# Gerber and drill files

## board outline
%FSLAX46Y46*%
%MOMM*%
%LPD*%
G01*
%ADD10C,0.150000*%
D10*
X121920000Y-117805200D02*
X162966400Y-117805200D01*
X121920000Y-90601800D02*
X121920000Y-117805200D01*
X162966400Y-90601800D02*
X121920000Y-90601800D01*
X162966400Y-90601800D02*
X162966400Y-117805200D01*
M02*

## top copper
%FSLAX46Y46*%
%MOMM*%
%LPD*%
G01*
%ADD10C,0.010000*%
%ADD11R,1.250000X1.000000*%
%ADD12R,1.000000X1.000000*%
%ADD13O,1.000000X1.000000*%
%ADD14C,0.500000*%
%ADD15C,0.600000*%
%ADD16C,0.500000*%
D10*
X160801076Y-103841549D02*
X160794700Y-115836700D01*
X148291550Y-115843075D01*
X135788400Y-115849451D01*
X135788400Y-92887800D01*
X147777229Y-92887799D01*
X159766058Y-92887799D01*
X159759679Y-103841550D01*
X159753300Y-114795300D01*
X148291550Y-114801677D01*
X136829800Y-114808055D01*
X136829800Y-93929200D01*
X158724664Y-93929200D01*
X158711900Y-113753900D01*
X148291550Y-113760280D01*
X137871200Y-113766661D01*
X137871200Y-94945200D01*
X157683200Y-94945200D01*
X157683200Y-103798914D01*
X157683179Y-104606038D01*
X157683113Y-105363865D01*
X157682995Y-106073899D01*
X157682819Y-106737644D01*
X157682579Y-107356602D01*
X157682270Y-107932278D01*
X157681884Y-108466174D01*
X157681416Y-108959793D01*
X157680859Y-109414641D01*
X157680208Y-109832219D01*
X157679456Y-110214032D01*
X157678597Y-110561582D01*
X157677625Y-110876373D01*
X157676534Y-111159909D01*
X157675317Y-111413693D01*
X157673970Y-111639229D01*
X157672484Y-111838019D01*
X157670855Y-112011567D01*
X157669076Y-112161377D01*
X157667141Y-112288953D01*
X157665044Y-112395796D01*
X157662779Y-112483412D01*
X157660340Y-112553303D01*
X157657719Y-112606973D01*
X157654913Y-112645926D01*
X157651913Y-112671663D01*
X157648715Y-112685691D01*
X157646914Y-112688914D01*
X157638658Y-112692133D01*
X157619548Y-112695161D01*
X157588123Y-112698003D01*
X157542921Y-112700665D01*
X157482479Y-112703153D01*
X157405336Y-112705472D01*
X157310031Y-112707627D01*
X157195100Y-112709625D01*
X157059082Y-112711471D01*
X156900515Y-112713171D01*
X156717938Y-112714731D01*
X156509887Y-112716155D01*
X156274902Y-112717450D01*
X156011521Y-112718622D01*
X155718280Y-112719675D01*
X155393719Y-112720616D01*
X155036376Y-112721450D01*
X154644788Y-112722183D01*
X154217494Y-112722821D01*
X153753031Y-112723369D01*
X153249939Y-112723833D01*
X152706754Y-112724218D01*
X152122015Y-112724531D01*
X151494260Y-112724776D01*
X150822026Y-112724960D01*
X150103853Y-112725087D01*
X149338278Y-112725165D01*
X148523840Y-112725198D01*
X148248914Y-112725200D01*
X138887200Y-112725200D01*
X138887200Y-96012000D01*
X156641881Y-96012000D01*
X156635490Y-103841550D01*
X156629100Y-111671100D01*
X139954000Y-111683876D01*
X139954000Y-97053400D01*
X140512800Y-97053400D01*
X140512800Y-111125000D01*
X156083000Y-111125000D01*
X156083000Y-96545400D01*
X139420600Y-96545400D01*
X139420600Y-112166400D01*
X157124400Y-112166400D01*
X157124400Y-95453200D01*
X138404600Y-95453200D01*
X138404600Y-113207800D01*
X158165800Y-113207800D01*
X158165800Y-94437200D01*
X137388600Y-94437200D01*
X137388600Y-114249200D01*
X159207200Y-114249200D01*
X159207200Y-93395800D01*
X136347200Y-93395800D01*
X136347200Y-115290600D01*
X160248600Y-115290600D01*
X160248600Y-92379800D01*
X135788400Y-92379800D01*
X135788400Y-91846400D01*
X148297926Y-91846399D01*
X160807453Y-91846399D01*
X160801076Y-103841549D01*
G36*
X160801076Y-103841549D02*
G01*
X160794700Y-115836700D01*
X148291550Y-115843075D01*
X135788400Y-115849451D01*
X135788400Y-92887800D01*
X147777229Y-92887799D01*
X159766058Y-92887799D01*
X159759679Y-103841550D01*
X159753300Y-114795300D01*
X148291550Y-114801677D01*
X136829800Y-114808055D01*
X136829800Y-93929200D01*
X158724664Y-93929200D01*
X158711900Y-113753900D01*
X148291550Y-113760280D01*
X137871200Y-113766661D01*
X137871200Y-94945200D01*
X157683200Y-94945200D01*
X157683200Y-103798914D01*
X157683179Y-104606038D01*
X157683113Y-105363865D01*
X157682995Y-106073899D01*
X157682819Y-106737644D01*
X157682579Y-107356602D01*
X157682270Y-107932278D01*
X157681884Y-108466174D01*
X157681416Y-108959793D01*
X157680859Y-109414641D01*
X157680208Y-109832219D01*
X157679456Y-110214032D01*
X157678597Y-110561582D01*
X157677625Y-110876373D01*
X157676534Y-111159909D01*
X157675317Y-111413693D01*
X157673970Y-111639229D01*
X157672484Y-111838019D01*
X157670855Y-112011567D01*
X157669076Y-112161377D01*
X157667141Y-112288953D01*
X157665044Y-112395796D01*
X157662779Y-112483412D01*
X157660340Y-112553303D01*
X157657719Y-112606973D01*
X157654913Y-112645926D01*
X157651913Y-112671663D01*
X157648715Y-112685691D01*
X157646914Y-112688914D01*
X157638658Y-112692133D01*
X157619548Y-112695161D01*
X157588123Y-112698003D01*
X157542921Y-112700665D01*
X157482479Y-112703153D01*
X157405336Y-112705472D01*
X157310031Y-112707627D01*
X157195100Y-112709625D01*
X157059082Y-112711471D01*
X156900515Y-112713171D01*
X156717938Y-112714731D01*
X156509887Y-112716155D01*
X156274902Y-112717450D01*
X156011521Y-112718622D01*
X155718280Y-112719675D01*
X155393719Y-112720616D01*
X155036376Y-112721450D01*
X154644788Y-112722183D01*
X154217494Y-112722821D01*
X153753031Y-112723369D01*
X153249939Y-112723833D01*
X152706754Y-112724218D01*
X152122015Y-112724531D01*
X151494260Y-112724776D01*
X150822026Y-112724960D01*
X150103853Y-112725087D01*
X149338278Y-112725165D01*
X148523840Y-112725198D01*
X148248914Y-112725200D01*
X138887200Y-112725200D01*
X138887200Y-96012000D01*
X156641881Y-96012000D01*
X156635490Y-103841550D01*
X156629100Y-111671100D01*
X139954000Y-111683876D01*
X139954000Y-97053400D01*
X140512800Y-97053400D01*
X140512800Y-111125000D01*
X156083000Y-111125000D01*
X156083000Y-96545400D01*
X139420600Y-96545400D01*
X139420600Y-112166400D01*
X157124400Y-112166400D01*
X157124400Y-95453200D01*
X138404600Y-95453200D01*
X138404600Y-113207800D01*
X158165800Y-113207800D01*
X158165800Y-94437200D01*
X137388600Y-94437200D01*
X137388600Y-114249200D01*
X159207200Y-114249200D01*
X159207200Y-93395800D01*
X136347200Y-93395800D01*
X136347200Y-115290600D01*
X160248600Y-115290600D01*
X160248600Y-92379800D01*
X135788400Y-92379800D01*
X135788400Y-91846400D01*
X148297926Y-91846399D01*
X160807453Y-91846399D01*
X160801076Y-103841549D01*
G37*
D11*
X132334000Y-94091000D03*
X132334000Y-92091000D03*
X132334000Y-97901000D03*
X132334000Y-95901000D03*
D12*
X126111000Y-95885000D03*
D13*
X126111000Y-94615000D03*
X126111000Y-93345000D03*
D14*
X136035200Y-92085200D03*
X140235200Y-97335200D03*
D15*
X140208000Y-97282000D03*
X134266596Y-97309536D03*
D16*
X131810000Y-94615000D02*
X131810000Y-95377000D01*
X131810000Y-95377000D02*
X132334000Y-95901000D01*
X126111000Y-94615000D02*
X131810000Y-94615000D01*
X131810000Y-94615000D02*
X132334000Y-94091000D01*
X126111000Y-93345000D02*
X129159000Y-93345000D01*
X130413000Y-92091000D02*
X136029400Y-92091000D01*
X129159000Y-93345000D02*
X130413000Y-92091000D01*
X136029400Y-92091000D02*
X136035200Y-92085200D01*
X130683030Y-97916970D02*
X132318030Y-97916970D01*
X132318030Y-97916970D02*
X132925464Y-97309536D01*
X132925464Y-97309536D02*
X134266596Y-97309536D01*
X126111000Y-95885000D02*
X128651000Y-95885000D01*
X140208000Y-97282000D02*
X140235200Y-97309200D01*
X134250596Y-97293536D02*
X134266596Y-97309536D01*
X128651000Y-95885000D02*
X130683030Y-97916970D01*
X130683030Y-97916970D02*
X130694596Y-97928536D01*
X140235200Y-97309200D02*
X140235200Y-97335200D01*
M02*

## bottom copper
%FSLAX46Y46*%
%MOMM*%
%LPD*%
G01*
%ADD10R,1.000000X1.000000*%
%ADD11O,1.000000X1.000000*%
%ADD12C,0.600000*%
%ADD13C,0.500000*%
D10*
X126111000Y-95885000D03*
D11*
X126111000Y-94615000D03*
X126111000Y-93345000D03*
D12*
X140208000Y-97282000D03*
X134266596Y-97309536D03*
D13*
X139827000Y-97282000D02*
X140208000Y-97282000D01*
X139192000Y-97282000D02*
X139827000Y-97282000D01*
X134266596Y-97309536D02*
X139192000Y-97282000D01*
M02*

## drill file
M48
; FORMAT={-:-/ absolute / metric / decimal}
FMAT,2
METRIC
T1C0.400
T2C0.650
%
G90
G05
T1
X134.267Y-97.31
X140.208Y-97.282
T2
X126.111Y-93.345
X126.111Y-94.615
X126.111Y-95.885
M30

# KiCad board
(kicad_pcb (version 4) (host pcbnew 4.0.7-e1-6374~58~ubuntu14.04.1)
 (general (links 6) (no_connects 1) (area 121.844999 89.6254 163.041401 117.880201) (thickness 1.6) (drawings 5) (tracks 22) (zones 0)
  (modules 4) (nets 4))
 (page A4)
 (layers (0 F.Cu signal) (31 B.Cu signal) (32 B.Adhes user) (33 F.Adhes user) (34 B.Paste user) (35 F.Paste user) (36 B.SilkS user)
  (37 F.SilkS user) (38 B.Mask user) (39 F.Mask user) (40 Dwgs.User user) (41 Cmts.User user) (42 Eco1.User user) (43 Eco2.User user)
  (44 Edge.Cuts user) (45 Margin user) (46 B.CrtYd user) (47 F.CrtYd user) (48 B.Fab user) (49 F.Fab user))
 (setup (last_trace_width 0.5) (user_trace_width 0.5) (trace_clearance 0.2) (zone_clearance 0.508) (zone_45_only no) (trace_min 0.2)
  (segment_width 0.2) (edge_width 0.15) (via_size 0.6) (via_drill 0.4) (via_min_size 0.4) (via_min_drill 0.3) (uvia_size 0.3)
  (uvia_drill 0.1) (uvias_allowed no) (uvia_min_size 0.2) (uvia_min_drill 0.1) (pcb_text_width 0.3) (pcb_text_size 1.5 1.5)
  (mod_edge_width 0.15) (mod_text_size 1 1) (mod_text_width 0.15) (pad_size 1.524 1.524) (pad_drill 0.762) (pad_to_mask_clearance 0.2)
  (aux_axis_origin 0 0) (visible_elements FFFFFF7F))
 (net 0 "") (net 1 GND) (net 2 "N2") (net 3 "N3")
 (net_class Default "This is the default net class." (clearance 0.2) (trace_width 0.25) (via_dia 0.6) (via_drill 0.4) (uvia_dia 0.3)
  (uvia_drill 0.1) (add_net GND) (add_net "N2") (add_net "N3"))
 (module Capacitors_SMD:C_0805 (layer F.Cu) (at 132.334 93.091 90)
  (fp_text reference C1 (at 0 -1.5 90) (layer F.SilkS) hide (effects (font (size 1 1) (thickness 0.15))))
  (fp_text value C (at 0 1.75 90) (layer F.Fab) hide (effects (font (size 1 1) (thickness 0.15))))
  (pad 1 smd rect (at -1 0 90) (size 1 1.25) (layers F.Cu F.Paste F.Mask) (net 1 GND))
  (pad 2 smd rect (at 1 0 90) (size 1 1.25) (layers F.Cu F.Paste F.Mask) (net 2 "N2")))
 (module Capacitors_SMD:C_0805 (layer F.Cu) (at 132.334 96.901 90)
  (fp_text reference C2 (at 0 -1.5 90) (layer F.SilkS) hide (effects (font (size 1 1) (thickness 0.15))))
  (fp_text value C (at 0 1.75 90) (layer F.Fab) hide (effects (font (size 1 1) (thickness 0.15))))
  (pad 1 smd rect (at -1 0 90) (size 1 1.25) (layers F.Cu F.Paste F.Mask) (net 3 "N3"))
  (pad 2 smd rect (at 1 0 90) (size 1 1.25) (layers F.Cu F.Paste F.Mask) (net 1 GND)))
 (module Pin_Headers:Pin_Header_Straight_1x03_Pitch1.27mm (layer F.Cu) (at 126.111 95.885 180)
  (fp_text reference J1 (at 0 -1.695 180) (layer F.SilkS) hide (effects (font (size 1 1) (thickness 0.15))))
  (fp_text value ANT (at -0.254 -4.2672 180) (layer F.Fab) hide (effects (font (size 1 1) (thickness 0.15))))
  (pad 1 thru_hole rect (at 0 0 180) (size 1 1) (drill 0.65) (layers *.Cu *.Mask) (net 3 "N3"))
  (pad 2 thru_hole oval (at 0 1.27 180) (size 1 1) (drill 0.65) (layers *.Cu *.Mask) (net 1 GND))
  (pad 3 thru_hole oval (at 0 2.54 180) (size 1 1) (drill 0.65) (layers *.Cu *.Mask) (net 2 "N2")))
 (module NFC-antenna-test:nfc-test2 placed (layer F.Cu) (at 148.2852 103.8352)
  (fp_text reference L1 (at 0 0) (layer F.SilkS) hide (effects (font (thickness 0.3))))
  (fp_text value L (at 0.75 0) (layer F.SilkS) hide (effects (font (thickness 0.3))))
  (fp_poly
   (pts (xy 12.515876 0.006349) (xy 12.5095 12.0015) (xy 0.00635 12.007875) (xy -12.4968 12.014251) (xy -12.4968 -10.9474)
    (xy -0.507971 -10.947401) (xy 11.480858 -10.947401) (xy 11.474479 0.00635) (xy 11.4681 10.9601) (xy 0.00635 10.966477)
    (xy -11.4554 10.972855) (xy -11.4554 -9.906) (xy 10.439464 -9.906) (xy 10.4267 9.9187) (xy 0.00635 9.92508) (xy -10.414 9.931461)
    (xy -10.414 -8.89) (xy 9.398 -8.89) (xy 9.398 -0.036286) (xy 9.397979 0.770838) (xy 9.397913 1.528665) (xy 9.397795 2.238699)
    (xy 9.397619 2.902444) (xy 9.397379 3.521402) (xy 9.39707 4.097078) (xy 9.396684 4.630974) (xy 9.396216 5.124593) (xy 9.395659 5.579441)
    (xy 9.395008 5.997019) (xy 9.394256 6.378832) (xy 9.393397 6.726382) (xy 9.392425 7.041173) (xy 9.391334 7.324709)
    (xy 9.390117 7.578493) (xy 9.38877 7.804029) (xy 9.387284 8.002819) (xy 9.385655 8.176367) (xy 9.383876 8.326177) (xy 9.381941 8.453753)
    (xy 9.379844 8.560596) (xy 9.377579 8.648212) (xy 9.37514 8.718103) (xy 9.372519 8.771773) (xy 9.369713 8.810726) (xy 9.366713 8.836463)
    (xy 9.363515 8.850491) (xy 9.361714 8.853714) (xy 9.353458 8.856933) (xy 9.334348 8.859961) (xy 9.302923 8.862803)
    (xy 9.257721 8.865465) (xy 9.197279 8.867953) (xy 9.120136 8.870272) (xy 9.024831 8.872427) (xy 8.9099 8.874425) (xy 8.773882 8.876271)
    (xy 8.615315 8.877971) (xy 8.432738 8.879531) (xy 8.224687 8.880955) (xy 7.989702 8.88225) (xy 7.726321 8.883422) (xy 7.43308 8.884475)
    (xy 7.108519 8.885416) (xy 6.751176 8.88625) (xy 6.359588 8.886983) (xy 5.932294 8.887621) (xy 5.467831 8.888169) (xy 4.964739 8.888633)
    (xy 4.421554 8.889018) (xy 3.836815 8.889331) (xy 3.20906 8.889576) (xy 2.536826 8.88976) (xy 1.818653 8.889887) (xy 1.053078 8.889965)
    (xy 0.23864 8.889998) (xy -0.036286 8.89) (xy -9.398 8.89) (xy -9.398 -7.8232) (xy 8.356681 -7.8232) (xy 8.35029 0.00635)
    (xy 8.3439 7.8359) (xy -8.3312 7.848676) (xy -8.3312 -6.7818) (xy -7.7724 -6.7818) (xy -7.7724 7.2898) (xy 7.7978 7.2898)
    (xy 7.7978 -7.2898) (xy -8.8646 -7.2898) (xy -8.8646 8.3312) (xy 8.8392 8.3312) (xy 8.8392 -8.382) (xy -9.8806 -8.382)
    (xy -9.8806 9.3726) (xy 9.8806 9.3726) (xy 9.8806 -9.398) (xy -10.8966 -9.398) (xy -10.8966 10.414) (xy 10.922 10.414)
    (xy 10.922 -10.4394) (xy -11.938 -10.4394) (xy -11.938 11.4554) (xy 11.9634 11.4554) (xy 11.9634 -11.4554) (xy -12.4968 -11.4554)
    (xy -12.4968 -11.9888) (xy 0.012726 -11.988801) (xy 12.522253 -11.988801) (xy 12.515876 0.006349))
   (layer F.Cu) (width 0.01))
  (pad 1 smd circle (at -12.25 -11.75) (size 0.5 0.5) (layers F.Cu F.Paste F.Mask) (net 2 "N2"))
  (pad 2 smd circle (at -8.05 -6.5) (size 0.5 0.5) (layers F.Cu F.Paste F.Mask) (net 3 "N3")))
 (gr_line (start 121.92 117.8052) (end 162.9664 117.8052) (angle 90) (layer Edge.Cuts) (width 0.15))
 (gr_line (start 121.92 90.6018) (end 121.92 117.8052) (angle 90) (layer Edge.Cuts) (width 0.15))
 (gr_line (start 162.9664 90.6018) (end 121.92 90.6018) (angle 90) (layer Edge.Cuts) (width 0.15))
 (gr_line (start 162.9664 90.6018) (end 162.9664 117.8052) (angle 90) (layer Edge.Cuts) (width 0.15))
 (segment (start 131.81 94.615) (end 131.81 95.377) (width 0.5) (layer F.Cu) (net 1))
 (segment (start 131.81 95.377) (end 132.334 95.901) (width 0.5) (layer F.Cu) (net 1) (status 800000))
 (segment (start 126.111 94.615) (end 131.81 94.615) (width 0.5) (layer F.Cu) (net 1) (status 400000))
 (segment (start 131.81 94.615) (end 132.334 94.091) (width 0.5) (layer F.Cu) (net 1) (status 800000))
 (segment (start 126.111 93.345) (end 129.159 93.345) (width 0.5) (layer F.Cu) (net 2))
 (segment (start 130.413 92.091) (end 136.0294 92.091) (width 0.5) (layer F.Cu) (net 2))
 (segment (start 129.159 93.345) (end 130.413 92.091) (width 0.5) (layer F.Cu) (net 2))
 (segment (start 136.0294 92.091) (end 136.0352 92.0852) (width 0.5) (layer F.Cu) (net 2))
 (segment (start 130.68303 97.91697) (end 132.31803 97.91697) (width 0.5) (layer F.Cu) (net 3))
 (segment (start 132.31803 97.91697) (end 132.925464 97.309536) (width 0.5) (layer F.Cu) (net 3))
 (segment (start 132.925464 97.309536) (end 134.266596 97.309536) (width 0.5) (layer F.Cu) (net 3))
 (segment (start 126.111 95.885) (end 128.651 95.885) (width 0.5) (layer F.Cu) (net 3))
 (segment (start 140.208 97.282) (end 140.2352 97.3092) (width 0.5) (layer F.Cu) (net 3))
 (via (at 140.208 97.282) (size 0.6) (drill 0.4) (layers F.Cu B.Cu) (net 3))
 (segment (start 139.827 97.282) (end 140.208 97.282) (width 0.5) (layer B.Cu) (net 3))
 (segment (start 139.192 97.282) (end 139.827 97.282) (width 0.5) (layer B.Cu) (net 3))
 (segment (start 134.266596 97.309536) (end 139.192 97.282) (width 0.5) (layer B.Cu) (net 3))
 (via (at 134.266596 97.309536) (size 0.6) (drill 0.4) (layers F.Cu B.Cu) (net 3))
 (segment (start 134.250596 97.293536) (end 134.266596 97.309536) (width 0.5) (layer F.Cu) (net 3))
 (segment (start 128.651 95.885) (end 130.68303 97.91697) (width 0.5) (layer F.Cu) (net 3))
 (segment (start 130.68303 97.91697) (end 130.694596 97.928536) (width 0.5) (layer F.Cu) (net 3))
 (segment (start 140.2352 97.3092) (end 140.2352 97.3352) (width 0.5) (layer F.Cu) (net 3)))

